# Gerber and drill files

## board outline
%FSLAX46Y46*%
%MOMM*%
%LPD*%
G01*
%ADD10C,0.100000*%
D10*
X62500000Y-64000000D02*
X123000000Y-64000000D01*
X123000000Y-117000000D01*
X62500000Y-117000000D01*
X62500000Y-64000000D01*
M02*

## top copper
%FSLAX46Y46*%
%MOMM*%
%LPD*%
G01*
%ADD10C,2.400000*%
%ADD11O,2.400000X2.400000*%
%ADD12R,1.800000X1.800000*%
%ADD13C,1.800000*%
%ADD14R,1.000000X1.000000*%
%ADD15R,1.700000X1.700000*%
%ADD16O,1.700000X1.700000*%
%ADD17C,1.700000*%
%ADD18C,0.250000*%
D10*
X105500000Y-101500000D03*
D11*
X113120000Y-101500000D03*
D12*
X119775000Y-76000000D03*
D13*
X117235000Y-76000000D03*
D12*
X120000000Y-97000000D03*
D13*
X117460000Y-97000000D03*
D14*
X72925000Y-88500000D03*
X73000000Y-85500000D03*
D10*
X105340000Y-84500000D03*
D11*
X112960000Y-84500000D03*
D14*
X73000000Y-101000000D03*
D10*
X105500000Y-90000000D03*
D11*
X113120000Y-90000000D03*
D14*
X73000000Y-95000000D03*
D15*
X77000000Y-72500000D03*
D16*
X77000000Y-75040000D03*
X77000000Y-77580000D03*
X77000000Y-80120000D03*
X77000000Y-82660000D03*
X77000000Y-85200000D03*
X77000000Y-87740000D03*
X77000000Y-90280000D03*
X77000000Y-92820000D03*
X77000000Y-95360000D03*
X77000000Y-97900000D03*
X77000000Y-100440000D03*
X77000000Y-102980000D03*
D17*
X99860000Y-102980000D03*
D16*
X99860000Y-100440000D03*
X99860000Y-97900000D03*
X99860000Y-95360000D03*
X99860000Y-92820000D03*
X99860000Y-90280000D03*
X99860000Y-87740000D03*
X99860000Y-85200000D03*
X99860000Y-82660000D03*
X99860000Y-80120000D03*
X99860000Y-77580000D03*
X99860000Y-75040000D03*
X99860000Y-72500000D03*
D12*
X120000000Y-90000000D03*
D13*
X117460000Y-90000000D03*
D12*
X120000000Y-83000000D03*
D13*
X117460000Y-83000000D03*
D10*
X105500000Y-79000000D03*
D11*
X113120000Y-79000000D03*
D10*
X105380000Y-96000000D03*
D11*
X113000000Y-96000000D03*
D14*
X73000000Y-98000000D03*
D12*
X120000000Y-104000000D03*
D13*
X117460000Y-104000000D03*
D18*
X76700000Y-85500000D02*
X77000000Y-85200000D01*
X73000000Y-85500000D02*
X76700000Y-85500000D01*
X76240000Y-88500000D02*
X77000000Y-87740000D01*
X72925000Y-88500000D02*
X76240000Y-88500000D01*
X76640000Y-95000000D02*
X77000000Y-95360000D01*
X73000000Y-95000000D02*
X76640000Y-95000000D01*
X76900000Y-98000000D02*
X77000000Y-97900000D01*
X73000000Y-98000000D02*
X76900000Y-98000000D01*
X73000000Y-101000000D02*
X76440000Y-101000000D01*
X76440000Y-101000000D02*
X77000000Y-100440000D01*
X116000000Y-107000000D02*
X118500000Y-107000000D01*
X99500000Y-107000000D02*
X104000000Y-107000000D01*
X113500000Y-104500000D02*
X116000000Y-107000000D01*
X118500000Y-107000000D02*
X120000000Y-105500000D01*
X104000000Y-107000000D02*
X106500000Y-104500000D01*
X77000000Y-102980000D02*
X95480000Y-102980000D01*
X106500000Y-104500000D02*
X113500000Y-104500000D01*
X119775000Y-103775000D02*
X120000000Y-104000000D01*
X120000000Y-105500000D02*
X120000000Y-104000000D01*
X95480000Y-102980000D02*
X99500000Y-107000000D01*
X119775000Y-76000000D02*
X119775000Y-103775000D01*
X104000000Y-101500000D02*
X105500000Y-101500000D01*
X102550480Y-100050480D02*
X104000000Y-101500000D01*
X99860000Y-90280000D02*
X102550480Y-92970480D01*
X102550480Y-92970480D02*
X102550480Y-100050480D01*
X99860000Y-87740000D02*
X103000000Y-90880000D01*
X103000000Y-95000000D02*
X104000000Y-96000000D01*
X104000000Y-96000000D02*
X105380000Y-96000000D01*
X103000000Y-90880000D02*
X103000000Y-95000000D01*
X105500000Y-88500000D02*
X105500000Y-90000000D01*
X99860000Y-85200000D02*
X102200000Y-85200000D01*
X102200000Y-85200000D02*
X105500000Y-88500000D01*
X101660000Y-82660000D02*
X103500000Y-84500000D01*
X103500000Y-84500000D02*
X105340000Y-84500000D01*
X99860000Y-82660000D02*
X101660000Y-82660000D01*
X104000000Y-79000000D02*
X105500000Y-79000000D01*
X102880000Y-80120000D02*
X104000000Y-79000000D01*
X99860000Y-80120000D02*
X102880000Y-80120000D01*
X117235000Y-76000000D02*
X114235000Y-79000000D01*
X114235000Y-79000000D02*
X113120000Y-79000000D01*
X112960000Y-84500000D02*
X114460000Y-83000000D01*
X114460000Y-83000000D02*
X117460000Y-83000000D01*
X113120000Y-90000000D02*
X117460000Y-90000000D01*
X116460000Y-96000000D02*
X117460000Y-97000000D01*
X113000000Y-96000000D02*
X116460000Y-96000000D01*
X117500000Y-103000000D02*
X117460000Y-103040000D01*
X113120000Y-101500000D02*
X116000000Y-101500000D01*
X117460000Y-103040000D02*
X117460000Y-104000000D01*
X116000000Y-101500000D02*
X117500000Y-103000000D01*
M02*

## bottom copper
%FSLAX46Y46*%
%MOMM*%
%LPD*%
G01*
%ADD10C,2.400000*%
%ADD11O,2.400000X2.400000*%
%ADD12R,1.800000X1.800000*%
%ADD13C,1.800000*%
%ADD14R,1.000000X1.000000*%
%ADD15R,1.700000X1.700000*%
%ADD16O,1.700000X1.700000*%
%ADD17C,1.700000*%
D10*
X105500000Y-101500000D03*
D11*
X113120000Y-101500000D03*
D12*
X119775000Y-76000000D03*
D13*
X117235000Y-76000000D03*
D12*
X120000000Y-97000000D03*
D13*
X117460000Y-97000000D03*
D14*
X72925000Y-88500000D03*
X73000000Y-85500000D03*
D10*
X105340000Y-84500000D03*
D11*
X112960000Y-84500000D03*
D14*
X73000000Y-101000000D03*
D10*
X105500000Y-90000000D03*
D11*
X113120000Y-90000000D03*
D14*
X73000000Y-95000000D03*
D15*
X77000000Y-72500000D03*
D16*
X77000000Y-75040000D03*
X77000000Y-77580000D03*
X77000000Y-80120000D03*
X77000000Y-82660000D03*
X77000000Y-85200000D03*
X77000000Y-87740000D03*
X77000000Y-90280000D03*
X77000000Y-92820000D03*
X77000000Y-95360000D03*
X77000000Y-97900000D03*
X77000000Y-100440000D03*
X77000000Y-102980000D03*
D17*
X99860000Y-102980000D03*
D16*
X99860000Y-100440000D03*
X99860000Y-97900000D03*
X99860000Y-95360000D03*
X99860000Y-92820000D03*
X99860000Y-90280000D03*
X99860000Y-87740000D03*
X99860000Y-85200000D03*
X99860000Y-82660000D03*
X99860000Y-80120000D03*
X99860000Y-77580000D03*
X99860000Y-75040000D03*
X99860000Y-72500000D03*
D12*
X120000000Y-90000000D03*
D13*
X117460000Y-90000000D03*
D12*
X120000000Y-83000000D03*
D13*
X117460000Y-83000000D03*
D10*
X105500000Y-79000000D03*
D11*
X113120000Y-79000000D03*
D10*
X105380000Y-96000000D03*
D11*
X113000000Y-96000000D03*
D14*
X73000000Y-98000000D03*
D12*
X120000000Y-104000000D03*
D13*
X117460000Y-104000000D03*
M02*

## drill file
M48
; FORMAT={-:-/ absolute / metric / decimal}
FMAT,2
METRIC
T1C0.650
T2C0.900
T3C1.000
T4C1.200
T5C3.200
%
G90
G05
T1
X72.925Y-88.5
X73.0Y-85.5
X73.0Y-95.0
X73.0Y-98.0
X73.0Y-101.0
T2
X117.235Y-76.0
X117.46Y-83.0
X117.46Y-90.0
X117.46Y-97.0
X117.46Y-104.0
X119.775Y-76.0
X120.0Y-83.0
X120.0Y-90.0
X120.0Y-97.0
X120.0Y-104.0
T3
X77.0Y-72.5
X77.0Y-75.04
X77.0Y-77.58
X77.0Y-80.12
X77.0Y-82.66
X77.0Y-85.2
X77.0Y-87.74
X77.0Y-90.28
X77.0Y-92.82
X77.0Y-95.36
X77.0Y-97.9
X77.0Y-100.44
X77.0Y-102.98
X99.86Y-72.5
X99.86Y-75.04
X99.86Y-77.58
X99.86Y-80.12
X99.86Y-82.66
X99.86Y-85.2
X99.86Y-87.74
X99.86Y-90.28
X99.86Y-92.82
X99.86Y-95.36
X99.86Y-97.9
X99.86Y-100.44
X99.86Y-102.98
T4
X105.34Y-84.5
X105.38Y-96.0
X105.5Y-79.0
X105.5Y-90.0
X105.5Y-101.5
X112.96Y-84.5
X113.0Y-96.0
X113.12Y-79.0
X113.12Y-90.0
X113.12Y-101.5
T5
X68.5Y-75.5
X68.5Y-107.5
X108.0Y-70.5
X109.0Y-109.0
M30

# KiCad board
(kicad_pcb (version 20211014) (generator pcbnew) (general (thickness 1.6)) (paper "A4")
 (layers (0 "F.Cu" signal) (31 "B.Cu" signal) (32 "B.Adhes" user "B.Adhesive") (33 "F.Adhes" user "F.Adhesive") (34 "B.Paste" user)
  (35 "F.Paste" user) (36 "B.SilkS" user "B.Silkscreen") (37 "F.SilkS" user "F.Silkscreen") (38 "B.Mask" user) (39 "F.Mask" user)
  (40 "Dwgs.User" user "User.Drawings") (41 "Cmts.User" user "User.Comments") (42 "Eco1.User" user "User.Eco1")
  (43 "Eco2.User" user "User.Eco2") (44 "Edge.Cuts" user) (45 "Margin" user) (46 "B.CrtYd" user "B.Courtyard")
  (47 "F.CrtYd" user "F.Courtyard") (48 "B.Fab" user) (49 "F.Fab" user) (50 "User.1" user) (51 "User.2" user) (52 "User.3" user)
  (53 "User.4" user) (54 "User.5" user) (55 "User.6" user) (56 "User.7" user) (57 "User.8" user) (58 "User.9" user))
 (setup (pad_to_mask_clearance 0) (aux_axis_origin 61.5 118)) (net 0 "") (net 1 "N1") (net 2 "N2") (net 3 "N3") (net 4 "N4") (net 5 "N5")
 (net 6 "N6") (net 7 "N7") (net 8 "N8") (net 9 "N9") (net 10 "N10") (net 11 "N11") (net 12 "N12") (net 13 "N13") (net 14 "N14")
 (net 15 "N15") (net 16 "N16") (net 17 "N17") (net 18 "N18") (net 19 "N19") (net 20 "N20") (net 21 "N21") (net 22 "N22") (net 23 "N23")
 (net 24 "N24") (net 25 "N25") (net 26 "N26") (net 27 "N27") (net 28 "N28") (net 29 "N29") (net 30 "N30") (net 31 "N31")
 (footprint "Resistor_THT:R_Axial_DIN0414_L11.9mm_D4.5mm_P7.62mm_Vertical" (layer "F.Cu") (at 105.5 101.5)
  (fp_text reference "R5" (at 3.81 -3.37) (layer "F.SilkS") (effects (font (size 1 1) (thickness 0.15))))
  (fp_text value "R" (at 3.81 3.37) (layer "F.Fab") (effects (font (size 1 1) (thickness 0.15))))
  (pad "1" thru_hole circle (at 0 0) (size 2.4 2.4) (drill 1.2) (layers *.Cu *.Mask) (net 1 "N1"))
  (pad "2" thru_hole oval (at 7.62 0) (size 2.4 2.4) (drill 1.2) (layers *.Cu *.Mask) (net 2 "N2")))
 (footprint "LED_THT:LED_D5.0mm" (layer "F.Cu") (at 119.775 76 180)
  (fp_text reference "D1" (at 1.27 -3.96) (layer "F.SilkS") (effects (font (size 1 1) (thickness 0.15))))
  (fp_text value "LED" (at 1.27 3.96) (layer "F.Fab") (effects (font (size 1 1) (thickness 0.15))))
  (pad "1" thru_hole rect (at 0 0 180) (size 1.8 1.8) (drill 0.9) (layers *.Cu *.Mask) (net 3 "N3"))
  (pad "2" thru_hole circle (at 2.54 0 180) (size 1.8 1.8) (drill 0.9) (layers *.Cu *.Mask) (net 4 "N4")))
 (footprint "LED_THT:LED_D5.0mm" (layer "F.Cu") (at 120 97 180)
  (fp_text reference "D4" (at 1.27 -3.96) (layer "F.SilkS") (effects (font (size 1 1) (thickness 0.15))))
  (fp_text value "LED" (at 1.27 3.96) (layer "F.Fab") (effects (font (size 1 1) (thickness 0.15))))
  (pad "1" thru_hole rect (at 0 0 180) (size 1.8 1.8) (drill 0.9) (layers *.Cu *.Mask) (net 3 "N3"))
  (pad "2" thru_hole circle (at 2.54 0 180) (size 1.8 1.8) (drill 0.9) (layers *.Cu *.Mask) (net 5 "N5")))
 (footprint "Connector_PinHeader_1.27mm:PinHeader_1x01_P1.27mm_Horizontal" (layer "F.Cu") (at 72.925 88.5 180)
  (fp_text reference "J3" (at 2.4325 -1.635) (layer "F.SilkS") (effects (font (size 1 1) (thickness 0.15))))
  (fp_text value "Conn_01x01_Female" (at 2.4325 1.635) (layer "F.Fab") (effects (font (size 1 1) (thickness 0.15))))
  (pad "1" thru_hole rect (at 0 0 180) (size 1 1) (drill 0.65) (layers *.Cu *.Mask) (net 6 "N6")))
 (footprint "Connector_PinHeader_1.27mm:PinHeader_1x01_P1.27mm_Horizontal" (layer "F.Cu") (at 73 85.5 180)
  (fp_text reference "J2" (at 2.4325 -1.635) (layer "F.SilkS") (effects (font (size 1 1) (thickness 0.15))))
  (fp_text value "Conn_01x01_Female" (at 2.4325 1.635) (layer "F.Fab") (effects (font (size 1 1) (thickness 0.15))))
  (pad "1" thru_hole rect (at 0 0 180) (size 1 1) (drill 0.65) (layers *.Cu *.Mask) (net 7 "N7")))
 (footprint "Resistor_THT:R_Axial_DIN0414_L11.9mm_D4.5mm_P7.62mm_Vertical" (layer "F.Cu") (at 105.34 84.5)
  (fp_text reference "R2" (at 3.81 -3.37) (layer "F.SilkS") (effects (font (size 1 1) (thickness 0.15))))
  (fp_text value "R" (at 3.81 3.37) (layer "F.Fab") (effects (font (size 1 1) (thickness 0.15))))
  (pad "1" thru_hole circle (at 0 0) (size 2.4 2.4) (drill 1.2) (layers *.Cu *.Mask) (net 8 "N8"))
  (pad "2" thru_hole oval (at 7.62 0) (size 2.4 2.4) (drill 1.2) (layers *.Cu *.Mask) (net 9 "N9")))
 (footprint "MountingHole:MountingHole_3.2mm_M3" (layer "F.Cu") (at 108 70.5)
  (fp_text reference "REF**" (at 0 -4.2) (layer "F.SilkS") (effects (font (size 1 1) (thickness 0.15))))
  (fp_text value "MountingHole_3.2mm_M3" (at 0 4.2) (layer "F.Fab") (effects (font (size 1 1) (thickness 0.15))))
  (pad "" np_thru_hole circle (at 0 0) (size 3.2 3.2) (drill 3.2) (layers *.Cu *.Mask)))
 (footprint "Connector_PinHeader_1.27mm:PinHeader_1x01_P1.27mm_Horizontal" (layer "F.Cu") (at 73 101 180)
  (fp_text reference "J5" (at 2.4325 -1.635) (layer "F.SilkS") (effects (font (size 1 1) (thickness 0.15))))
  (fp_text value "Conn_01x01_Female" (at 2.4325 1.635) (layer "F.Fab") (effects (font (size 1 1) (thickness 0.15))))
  (pad "1" thru_hole rect (at 0 0 180) (size 1 1) (drill 0.65) (layers *.Cu *.Mask) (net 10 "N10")))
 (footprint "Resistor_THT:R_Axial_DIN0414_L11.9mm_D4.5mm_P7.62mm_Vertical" (layer "F.Cu") (at 105.5 90)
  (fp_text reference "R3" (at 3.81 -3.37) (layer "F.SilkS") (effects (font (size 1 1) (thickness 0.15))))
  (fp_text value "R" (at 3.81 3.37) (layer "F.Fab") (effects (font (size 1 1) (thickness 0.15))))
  (pad "1" thru_hole circle (at 0 0) (size 2.4 2.4) (drill 1.2) (layers *.Cu *.Mask) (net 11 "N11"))
  (pad "2" thru_hole oval (at 7.62 0) (size 2.4 2.4) (drill 1.2) (layers *.Cu *.Mask) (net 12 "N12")))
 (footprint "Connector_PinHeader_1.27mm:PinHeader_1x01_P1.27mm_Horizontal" (layer "F.Cu") (at 73 95 180)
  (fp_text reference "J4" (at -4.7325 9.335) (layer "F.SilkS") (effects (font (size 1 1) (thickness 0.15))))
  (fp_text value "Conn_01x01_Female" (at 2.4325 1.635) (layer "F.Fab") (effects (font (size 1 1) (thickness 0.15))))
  (pad "1" thru_hole rect (at 0 0 180) (size 1 1) (drill 0.65) (layers *.Cu *.Mask) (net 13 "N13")))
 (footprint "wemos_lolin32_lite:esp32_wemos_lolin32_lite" (layer "F.Cu") (at 77 72.5)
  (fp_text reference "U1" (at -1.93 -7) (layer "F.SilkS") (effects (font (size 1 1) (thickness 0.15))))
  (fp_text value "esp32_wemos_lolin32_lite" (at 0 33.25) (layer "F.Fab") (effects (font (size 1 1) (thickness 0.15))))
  (pad "1" thru_hole rect (at 0 0) (size 1.7 1.7) (drill 1) (layers *.Cu *.Mask) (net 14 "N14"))
  (pad "2" thru_hole oval (at 0 2.54) (size 1.7 1.7) (drill 1) (layers *.Cu *.Mask) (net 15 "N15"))
  (pad "3" thru_hole oval (at 0 5.08) (size 1.7 1.7) (drill 1) (layers *.Cu *.Mask) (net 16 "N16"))
  (pad "4" thru_hole oval (at 0 7.62) (size 1.7 1.7) (drill 1) (layers *.Cu *.Mask) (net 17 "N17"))
  (pad "5" thru_hole oval (at 0 10.16) (size 1.7 1.7) (drill 1) (layers *.Cu *.Mask) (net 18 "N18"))
  (pad "6" thru_hole oval (at 0 12.7) (size 1.7 1.7) (drill 1) (layers *.Cu *.Mask) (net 7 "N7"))
  (pad "7" thru_hole oval (at 0 15.24) (size 1.7 1.7) (drill 1) (layers *.Cu *.Mask) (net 6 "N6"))
  (pad "8" thru_hole oval (at 0 17.78) (size 1.7 1.7) (drill 1) (layers *.Cu *.Mask) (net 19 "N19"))
  (pad "9" thru_hole oval (at 0 20.32) (size 1.7 1.7) (drill 1) (layers *.Cu *.Mask) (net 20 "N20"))
  (pad "10" thru_hole oval (at 0 22.86) (size 1.7 1.7) (drill 1) (layers *.Cu *.Mask) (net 13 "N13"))
  (pad "11" thru_hole oval (at 0 25.4) (size 1.7 1.7) (drill 1) (layers *.Cu *.Mask) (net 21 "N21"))
  (pad "12" thru_hole oval (at 0 27.94) (size 1.7 1.7) (drill 1) (layers *.Cu *.Mask) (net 10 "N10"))
  (pad "13" thru_hole oval (at 0 30.48) (size 1.7 1.7) (drill 1) (layers *.Cu *.Mask) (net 3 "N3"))
  (pad "14" thru_hole circle (at 22.86 30.48 180) (size 1.7 1.7) (drill 1) (layers *.Cu *.Mask) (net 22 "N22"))
  (pad "15" thru_hole oval (at 22.86 27.94 180) (size 1.7 1.7) (drill 1) (layers *.Cu *.Mask) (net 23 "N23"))
  (pad "16" thru_hole oval (at 22.86 25.4 180) (size 1.7 1.7) (drill 1) (layers *.Cu *.Mask) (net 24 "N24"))
  (pad "17" thru_hole oval (at 22.86 22.86 180) (size 1.7 1.7) (drill 1) (layers *.Cu *.Mask) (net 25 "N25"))
  (pad "18" thru_hole oval (at 22.86 20.32 180) (size 1.7 1.7) (drill 1) (layers *.Cu *.Mask) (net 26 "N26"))
  (pad "19" thru_hole oval (at 22.86 17.78 180) (size 1.7 1.7) (drill 1) (layers *.Cu *.Mask) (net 1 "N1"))
  (pad "20" thru_hole oval (at 22.86 15.24 180) (size 1.7 1.7) (drill 1) (layers *.Cu *.Mask) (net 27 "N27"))
  (pad "21" thru_hole oval (at 22.86 12.7 180) (size 1.7 1.7) (drill 1) (layers *.Cu *.Mask) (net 11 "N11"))
  (pad "22" thru_hole oval (at 22.86 10.16 180) (size 1.7 1.7) (drill 1) (layers *.Cu *.Mask) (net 8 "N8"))
  (pad "23" thru_hole oval (at 22.86 7.62 180) (size 1.7 1.7) (drill 1) (layers *.Cu *.Mask) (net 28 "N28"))
  (pad "24" thru_hole oval (at 22.86 5.08 180) (size 1.7 1.7) (drill 1) (layers *.Cu *.Mask) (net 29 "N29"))
  (pad "25" thru_hole oval (at 22.86 2.54 180) (size 1.7 1.7) (drill 1) (layers *.Cu *.Mask) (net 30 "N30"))
  (pad "26" thru_hole oval (at 22.86 0 180) (size 1.7 1.7) (drill 1) (layers *.Cu *.Mask) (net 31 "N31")))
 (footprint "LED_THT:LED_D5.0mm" (layer "F.Cu") (at 120 90 180)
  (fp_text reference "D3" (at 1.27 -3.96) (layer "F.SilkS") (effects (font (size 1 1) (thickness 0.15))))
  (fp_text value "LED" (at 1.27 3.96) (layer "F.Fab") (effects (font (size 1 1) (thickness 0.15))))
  (pad "1" thru_hole rect (at 0 0 180) (size 1.8 1.8) (drill 0.9) (layers *.Cu *.Mask) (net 3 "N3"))
  (pad "2" thru_hole circle (at 2.54 0 180) (size 1.8 1.8) (drill 0.9) (layers *.Cu *.Mask) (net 12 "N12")))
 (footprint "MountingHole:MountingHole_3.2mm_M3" (layer "F.Cu") (at 109 109)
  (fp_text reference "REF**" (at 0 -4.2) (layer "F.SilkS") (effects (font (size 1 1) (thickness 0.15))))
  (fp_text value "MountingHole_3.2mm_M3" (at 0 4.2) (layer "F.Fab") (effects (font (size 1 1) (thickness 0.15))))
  (pad "" np_thru_hole circle (at 0 0) (size 3.2 3.2) (drill 3.2) (layers *.Cu *.Mask)))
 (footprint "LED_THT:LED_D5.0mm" (layer "F.Cu") (at 120 83 180)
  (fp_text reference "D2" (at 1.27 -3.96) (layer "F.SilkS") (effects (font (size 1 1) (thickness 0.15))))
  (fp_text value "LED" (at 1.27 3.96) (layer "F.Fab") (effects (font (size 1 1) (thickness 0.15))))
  (pad "1" thru_hole rect (at 0 0 180) (size 1.8 1.8) (drill 0.9) (layers *.Cu *.Mask) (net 3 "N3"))
  (pad "2" thru_hole circle (at 2.54 0 180) (size 1.8 1.8) (drill 0.9) (layers *.Cu *.Mask) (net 9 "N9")))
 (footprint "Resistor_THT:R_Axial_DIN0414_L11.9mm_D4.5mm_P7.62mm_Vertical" (layer "F.Cu") (at 105.5 79)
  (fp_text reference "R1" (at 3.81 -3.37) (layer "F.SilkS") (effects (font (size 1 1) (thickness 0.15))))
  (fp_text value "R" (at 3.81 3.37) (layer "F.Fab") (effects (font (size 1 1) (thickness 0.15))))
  (pad "1" thru_hole circle (at 0 0) (size 2.4 2.4) (drill 1.2) (layers *.Cu *.Mask) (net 28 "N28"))
  (pad "2" thru_hole oval (at 7.62 0) (size 2.4 2.4) (drill 1.2) (layers *.Cu *.Mask) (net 4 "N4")))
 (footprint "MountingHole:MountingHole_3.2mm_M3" (layer "F.Cu") (at 68.5 75.5)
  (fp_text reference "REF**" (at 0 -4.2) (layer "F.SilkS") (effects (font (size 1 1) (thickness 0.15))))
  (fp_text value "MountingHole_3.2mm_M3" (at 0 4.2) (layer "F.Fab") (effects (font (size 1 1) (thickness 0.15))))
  (pad "" np_thru_hole circle (at 0 0) (size 3.2 3.2) (drill 3.2) (layers *.Cu *.Mask)))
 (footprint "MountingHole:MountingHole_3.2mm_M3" (layer "F.Cu") (at 68.5 107.5)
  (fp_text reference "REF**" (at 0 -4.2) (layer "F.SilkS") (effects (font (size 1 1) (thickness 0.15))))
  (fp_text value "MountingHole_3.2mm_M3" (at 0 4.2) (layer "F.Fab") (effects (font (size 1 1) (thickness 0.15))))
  (pad "" np_thru_hole circle (at 0 0) (size 3.2 3.2) (drill 3.2) (layers *.Cu *.Mask)))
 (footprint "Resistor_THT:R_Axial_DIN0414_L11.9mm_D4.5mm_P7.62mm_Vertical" (layer "F.Cu") (at 105.38 96)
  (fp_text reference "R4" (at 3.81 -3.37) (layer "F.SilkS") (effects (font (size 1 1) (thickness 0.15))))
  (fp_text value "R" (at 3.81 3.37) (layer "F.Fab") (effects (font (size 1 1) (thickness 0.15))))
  (pad "1" thru_hole circle (at 0 0) (size 2.4 2.4) (drill 1.2) (layers *.Cu *.Mask) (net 27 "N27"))
  (pad "2" thru_hole oval (at 7.62 0) (size 2.4 2.4) (drill 1.2) (layers *.Cu *.Mask) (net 5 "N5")))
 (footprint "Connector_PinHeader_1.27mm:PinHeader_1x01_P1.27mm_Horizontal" (layer "F.Cu") (at 73 98 180)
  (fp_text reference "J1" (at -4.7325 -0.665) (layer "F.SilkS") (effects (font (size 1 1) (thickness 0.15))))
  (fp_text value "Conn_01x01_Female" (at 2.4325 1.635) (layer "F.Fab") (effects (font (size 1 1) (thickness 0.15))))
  (pad "1" thru_hole rect (at 0 0 180) (size 1 1) (drill 0.65) (layers *.Cu *.Mask) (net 21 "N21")))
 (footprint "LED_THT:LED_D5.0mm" (layer "F.Cu") (at 120 104 180)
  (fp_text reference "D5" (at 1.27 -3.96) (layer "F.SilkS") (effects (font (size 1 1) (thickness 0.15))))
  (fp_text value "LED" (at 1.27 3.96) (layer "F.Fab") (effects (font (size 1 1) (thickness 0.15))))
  (pad "1" thru_hole rect (at 0 0 180) (size 1.8 1.8) (drill 0.9) (layers *.Cu *.Mask) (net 3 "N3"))
  (pad "2" thru_hole circle (at 2.54 0 180) (size 1.8 1.8) (drill 0.9) (layers *.Cu *.Mask) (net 2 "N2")))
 (gr_rect (start 62.5 64) (end 123 117) (layer "Edge.Cuts") (width 0.1) (fill none))
 (segment (start 76.7 85.5) (end 77 85.2) (width 0.25) (layer "F.Cu") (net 7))
 (segment (start 73 85.5) (end 76.7 85.5) (width 0.25) (layer "F.Cu") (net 7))
 (segment (start 76.24 88.5) (end 77 87.74) (width 0.25) (layer "F.Cu") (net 6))
 (segment (start 72.925 88.5) (end 76.24 88.5) (width 0.25) (layer "F.Cu") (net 6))
 (segment (start 76.64 95) (end 77 95.36) (width 0.25) (layer "F.Cu") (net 13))
 (segment (start 73 95) (end 76.64 95) (width 0.25) (layer "F.Cu") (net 13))
 (segment (start 76.9 98) (end 77 97.9) (width 0.25) (layer "F.Cu") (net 21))
 (segment (start 73 98) (end 76.9 98) (width 0.25) (layer "F.Cu") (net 21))
 (segment (start 73 101) (end 76.44 101) (width 0.25) (layer "F.Cu") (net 10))
 (segment (start 76.44 101) (end 77 100.44) (width 0.25) (layer "F.Cu") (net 10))
 (segment (start 116 107) (end 118.5 107) (width 0.25) (layer "F.Cu") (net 3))
 (segment (start 99.5 107) (end 104 107) (width 0.25) (layer "F.Cu") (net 3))
 (segment (start 113.5 104.5) (end 116 107) (width 0.25) (layer "F.Cu") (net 3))
 (segment (start 118.5 107) (end 120 105.5) (width 0.25) (layer "F.Cu") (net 3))
 (segment (start 104 107) (end 106.5 104.5) (width 0.25) (layer "F.Cu") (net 3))
 (segment (start 77 102.98) (end 95.48 102.98) (width 0.25) (layer "F.Cu") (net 3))
 (segment (start 106.5 104.5) (end 113.5 104.5) (width 0.25) (layer "F.Cu") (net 3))
 (segment (start 119.775 103.775) (end 120 104) (width 0.25) (layer "F.Cu") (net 3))
 (segment (start 120 105.5) (end 120 104) (width 0.25) (layer "F.Cu") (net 3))
 (segment (start 95.48 102.98) (end 99.5 107) (width 0.25) (layer "F.Cu") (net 3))
 (segment (start 119.775 76) (end 119.775 103.775) (width 0.25) (layer "F.Cu") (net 3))
 (segment (start 104 101.5) (end 105.5 101.5) (width 0.25) (layer "F.Cu") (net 1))
 (segment (start 102.55048 100.05048) (end 104 101.5) (width 0.25) (layer "F.Cu") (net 1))
 (segment (start 99.86 90.28) (end 102.55048 92.97048) (width 0.25) (layer "F.Cu") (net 1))
 (segment (start 102.55048 92.97048) (end 102.55048 100.05048) (width 0.25) (layer "F.Cu") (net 1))
 (segment (start 99.86 87.74) (end 103 90.88) (width 0.25) (layer "F.Cu") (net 27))
 (segment (start 103 95) (end 104 96) (width 0.25) (layer "F.Cu") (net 27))
 (segment (start 104 96) (end 105.38 96) (width 0.25) (layer "F.Cu") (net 27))
 (segment (start 103 90.88) (end 103 95) (width 0.25) (layer "F.Cu") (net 27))
 (segment (start 105.5 88.5) (end 105.5 90) (width 0.25) (layer "F.Cu") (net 11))
 (segment (start 99.86 85.2) (end 102.2 85.2) (width 0.25) (layer "F.Cu") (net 11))
 (segment (start 102.2 85.2) (end 105.5 88.5) (width 0.25) (layer "F.Cu") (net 11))
 (segment (start 101.66 82.66) (end 103.5 84.5) (width 0.25) (layer "F.Cu") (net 8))
 (segment (start 103.5 84.5) (end 105.34 84.5) (width 0.25) (layer "F.Cu") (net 8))
 (segment (start 99.86 82.66) (end 101.66 82.66) (width 0.25) (layer "F.Cu") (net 8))
 (segment (start 104 79) (end 105.5 79) (width 0.25) (layer "F.Cu") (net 28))
 (segment (start 102.88 80.12) (end 104 79) (width 0.25) (layer "F.Cu") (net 28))
 (segment (start 99.86 80.12) (end 102.88 80.12) (width 0.25) (layer "F.Cu") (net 28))
 (segment (start 117.235 76) (end 114.235 79) (width 0.25) (layer "F.Cu") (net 4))
 (segment (start 114.235 79) (end 113.12 79) (width 0.25) (layer "F.Cu") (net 4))
 (segment (start 112.96 84.5) (end 114.46 83) (width 0.25) (layer "F.Cu") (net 9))
 (segment (start 114.46 83) (end 117.46 83) (width 0.25) (layer "F.Cu") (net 9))
 (segment (start 113.12 90) (end 117.46 90) (width 0.25) (layer "F.Cu") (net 12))
 (segment (start 116.46 96) (end 117.46 97) (width 0.25) (layer "F.Cu") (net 5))
 (segment (start 113 96) (end 116.46 96) (width 0.25) (layer "F.Cu") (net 5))
 (segment (start 117.5 103) (end 117.46 103.04) (width 0.25) (layer "F.Cu") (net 2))
 (segment (start 113.12 101.5) (end 116 101.5) (width 0.25) (layer "F.Cu") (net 2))
 (segment (start 117.46 103.04) (end 117.46 104) (width 0.25) (layer "F.Cu") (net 2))
 (segment (start 116 101.5) (end 117.5 103) (width 0.25) (layer "F.Cu") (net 2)))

